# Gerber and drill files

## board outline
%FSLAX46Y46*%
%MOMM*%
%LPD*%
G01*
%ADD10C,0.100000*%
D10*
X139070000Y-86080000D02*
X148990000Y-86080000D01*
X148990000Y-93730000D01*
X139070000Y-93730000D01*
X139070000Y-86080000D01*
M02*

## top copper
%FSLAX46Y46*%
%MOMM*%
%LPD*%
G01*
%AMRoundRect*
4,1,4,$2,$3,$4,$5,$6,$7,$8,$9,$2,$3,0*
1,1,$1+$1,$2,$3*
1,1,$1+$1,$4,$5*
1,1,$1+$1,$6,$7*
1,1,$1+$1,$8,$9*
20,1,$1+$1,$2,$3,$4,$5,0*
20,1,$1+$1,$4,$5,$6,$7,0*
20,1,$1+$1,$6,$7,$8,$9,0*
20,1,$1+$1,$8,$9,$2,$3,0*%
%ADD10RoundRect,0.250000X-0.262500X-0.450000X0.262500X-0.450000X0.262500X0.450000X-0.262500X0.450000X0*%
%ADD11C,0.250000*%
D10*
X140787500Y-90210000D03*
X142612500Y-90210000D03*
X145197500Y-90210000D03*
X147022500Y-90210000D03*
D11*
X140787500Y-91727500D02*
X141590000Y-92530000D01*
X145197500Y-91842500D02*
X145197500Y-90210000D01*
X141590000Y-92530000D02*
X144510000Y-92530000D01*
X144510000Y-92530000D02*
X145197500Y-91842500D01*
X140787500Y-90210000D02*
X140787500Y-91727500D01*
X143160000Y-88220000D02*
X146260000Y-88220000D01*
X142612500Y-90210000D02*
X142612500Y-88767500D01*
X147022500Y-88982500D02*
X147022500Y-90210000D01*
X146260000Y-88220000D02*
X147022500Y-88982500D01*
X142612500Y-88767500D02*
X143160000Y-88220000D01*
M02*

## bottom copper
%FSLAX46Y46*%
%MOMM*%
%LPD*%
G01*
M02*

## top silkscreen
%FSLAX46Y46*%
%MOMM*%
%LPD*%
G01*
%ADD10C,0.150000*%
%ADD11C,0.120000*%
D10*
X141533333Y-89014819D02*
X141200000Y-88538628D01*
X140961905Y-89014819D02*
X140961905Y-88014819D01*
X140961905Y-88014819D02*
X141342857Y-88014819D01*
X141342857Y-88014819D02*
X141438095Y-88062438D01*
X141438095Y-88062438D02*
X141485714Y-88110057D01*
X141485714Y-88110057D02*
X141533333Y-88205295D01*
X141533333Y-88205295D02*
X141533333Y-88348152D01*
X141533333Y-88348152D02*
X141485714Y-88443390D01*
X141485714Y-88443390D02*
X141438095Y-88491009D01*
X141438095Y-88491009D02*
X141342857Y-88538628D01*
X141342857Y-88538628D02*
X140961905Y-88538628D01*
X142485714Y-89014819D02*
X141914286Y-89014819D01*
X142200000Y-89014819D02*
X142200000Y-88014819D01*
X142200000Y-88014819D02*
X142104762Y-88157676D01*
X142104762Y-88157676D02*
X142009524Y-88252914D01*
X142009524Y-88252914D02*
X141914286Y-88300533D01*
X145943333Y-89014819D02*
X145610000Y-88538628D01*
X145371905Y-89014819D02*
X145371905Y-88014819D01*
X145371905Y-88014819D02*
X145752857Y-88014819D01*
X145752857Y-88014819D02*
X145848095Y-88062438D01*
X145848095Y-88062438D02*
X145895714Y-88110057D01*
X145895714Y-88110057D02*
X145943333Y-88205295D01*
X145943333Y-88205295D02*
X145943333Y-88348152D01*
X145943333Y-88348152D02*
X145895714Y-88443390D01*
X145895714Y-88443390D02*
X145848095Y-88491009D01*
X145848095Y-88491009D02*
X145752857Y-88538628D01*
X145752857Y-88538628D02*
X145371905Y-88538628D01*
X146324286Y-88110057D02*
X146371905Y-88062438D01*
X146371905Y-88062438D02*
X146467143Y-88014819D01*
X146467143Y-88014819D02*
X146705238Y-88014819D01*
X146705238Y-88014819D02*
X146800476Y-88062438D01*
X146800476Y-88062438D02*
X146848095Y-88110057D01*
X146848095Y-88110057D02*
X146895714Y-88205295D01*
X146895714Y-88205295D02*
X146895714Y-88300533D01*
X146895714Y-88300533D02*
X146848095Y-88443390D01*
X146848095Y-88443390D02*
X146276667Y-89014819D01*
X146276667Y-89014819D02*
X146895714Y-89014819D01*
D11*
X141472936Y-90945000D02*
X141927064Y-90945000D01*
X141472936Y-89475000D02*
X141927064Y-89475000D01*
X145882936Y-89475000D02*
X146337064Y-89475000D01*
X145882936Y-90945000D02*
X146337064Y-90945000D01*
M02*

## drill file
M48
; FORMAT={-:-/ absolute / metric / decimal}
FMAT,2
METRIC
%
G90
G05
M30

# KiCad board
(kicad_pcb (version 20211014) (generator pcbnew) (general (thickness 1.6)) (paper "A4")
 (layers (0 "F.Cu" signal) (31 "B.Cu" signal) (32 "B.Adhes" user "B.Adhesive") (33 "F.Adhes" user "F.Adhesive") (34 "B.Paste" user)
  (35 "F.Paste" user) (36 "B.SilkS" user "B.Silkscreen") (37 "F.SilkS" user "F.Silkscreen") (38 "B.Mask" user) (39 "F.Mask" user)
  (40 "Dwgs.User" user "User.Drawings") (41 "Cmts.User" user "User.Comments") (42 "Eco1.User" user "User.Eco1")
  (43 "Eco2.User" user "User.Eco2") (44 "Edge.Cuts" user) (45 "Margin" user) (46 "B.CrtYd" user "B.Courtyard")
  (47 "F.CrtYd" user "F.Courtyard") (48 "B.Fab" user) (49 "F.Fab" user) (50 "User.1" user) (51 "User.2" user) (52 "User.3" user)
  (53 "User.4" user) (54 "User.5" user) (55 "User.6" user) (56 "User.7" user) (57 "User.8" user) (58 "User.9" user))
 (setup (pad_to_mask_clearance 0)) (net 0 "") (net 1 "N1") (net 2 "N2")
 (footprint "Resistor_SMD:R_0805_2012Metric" (layer "F.Cu") (at 141.7 90.21)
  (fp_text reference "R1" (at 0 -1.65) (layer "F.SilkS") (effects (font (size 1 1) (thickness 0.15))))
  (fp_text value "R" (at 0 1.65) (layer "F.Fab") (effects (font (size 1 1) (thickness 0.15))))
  (fp_line (start -0.227064 0.735) (end 0.227064 0.735) (layer "F.SilkS") (width 0.12))
  (fp_line (start -0.227064 -0.735) (end 0.227064 -0.735) (layer "F.SilkS") (width 0.12))
  (pad "1" smd roundrect (at -0.9125 0) (size 1.025 1.4) (layers "F.Cu" "F.Paste" "F.Mask") (roundrect_rratio 0.243902) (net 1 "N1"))
  (pad "2" smd roundrect (at 0.9125 0) (size 1.025 1.4) (layers "F.Cu" "F.Paste" "F.Mask") (roundrect_rratio 0.243902) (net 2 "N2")))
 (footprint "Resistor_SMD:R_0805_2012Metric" (layer "F.Cu") (at 146.11 90.21)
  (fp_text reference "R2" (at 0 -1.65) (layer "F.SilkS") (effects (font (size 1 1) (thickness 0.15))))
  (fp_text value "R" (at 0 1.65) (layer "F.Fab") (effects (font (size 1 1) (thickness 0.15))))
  (fp_line (start -0.227064 -0.735) (end 0.227064 -0.735) (layer "F.SilkS") (width 0.12))
  (fp_line (start -0.227064 0.735) (end 0.227064 0.735) (layer "F.SilkS") (width 0.12))
  (pad "1" smd roundrect (at -0.9125 0) (size 1.025 1.4) (layers "F.Cu" "F.Paste" "F.Mask") (roundrect_rratio 0.243902) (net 1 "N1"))
  (pad "2" smd roundrect (at 0.9125 0) (size 1.025 1.4) (layers "F.Cu" "F.Paste" "F.Mask") (roundrect_rratio 0.243902) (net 2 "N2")))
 (gr_rect (start 139.07 86.08) (end 148.99 93.73) (layer "Edge.Cuts") (width 0.1) (fill none))
 (segment (start 140.7875 91.7275) (end 141.59 92.53) (width 0.25) (layer "F.Cu") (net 1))
 (segment (start 145.1975 91.8425) (end 145.1975 90.21) (width 0.25) (layer "F.Cu") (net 1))
 (segment (start 141.59 92.53) (end 144.51 92.53) (width 0.25) (layer "F.Cu") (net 1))
 (segment (start 144.51 92.53) (end 145.1975 91.8425) (width 0.25) (layer "F.Cu") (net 1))
 (segment (start 140.7875 90.21) (end 140.7875 91.7275) (width 0.25) (layer "F.Cu") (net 1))
 (segment (start 143.16 88.22) (end 146.26 88.22) (width 0.25) (layer "F.Cu") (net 2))
 (segment (start 142.6125 90.21) (end 142.6125 88.7675) (width 0.25) (layer "F.Cu") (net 2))
 (segment (start 147.0225 88.9825) (end 147.0225 90.21) (width 0.25) (layer "F.Cu") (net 2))
 (segment (start 146.26 88.22) (end 147.0225 88.9825) (width 0.25) (layer "F.Cu") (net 2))
 (segment (start 142.6125 88.7675) (end 143.16 88.22) (width 0.25) (layer "F.Cu") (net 2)))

